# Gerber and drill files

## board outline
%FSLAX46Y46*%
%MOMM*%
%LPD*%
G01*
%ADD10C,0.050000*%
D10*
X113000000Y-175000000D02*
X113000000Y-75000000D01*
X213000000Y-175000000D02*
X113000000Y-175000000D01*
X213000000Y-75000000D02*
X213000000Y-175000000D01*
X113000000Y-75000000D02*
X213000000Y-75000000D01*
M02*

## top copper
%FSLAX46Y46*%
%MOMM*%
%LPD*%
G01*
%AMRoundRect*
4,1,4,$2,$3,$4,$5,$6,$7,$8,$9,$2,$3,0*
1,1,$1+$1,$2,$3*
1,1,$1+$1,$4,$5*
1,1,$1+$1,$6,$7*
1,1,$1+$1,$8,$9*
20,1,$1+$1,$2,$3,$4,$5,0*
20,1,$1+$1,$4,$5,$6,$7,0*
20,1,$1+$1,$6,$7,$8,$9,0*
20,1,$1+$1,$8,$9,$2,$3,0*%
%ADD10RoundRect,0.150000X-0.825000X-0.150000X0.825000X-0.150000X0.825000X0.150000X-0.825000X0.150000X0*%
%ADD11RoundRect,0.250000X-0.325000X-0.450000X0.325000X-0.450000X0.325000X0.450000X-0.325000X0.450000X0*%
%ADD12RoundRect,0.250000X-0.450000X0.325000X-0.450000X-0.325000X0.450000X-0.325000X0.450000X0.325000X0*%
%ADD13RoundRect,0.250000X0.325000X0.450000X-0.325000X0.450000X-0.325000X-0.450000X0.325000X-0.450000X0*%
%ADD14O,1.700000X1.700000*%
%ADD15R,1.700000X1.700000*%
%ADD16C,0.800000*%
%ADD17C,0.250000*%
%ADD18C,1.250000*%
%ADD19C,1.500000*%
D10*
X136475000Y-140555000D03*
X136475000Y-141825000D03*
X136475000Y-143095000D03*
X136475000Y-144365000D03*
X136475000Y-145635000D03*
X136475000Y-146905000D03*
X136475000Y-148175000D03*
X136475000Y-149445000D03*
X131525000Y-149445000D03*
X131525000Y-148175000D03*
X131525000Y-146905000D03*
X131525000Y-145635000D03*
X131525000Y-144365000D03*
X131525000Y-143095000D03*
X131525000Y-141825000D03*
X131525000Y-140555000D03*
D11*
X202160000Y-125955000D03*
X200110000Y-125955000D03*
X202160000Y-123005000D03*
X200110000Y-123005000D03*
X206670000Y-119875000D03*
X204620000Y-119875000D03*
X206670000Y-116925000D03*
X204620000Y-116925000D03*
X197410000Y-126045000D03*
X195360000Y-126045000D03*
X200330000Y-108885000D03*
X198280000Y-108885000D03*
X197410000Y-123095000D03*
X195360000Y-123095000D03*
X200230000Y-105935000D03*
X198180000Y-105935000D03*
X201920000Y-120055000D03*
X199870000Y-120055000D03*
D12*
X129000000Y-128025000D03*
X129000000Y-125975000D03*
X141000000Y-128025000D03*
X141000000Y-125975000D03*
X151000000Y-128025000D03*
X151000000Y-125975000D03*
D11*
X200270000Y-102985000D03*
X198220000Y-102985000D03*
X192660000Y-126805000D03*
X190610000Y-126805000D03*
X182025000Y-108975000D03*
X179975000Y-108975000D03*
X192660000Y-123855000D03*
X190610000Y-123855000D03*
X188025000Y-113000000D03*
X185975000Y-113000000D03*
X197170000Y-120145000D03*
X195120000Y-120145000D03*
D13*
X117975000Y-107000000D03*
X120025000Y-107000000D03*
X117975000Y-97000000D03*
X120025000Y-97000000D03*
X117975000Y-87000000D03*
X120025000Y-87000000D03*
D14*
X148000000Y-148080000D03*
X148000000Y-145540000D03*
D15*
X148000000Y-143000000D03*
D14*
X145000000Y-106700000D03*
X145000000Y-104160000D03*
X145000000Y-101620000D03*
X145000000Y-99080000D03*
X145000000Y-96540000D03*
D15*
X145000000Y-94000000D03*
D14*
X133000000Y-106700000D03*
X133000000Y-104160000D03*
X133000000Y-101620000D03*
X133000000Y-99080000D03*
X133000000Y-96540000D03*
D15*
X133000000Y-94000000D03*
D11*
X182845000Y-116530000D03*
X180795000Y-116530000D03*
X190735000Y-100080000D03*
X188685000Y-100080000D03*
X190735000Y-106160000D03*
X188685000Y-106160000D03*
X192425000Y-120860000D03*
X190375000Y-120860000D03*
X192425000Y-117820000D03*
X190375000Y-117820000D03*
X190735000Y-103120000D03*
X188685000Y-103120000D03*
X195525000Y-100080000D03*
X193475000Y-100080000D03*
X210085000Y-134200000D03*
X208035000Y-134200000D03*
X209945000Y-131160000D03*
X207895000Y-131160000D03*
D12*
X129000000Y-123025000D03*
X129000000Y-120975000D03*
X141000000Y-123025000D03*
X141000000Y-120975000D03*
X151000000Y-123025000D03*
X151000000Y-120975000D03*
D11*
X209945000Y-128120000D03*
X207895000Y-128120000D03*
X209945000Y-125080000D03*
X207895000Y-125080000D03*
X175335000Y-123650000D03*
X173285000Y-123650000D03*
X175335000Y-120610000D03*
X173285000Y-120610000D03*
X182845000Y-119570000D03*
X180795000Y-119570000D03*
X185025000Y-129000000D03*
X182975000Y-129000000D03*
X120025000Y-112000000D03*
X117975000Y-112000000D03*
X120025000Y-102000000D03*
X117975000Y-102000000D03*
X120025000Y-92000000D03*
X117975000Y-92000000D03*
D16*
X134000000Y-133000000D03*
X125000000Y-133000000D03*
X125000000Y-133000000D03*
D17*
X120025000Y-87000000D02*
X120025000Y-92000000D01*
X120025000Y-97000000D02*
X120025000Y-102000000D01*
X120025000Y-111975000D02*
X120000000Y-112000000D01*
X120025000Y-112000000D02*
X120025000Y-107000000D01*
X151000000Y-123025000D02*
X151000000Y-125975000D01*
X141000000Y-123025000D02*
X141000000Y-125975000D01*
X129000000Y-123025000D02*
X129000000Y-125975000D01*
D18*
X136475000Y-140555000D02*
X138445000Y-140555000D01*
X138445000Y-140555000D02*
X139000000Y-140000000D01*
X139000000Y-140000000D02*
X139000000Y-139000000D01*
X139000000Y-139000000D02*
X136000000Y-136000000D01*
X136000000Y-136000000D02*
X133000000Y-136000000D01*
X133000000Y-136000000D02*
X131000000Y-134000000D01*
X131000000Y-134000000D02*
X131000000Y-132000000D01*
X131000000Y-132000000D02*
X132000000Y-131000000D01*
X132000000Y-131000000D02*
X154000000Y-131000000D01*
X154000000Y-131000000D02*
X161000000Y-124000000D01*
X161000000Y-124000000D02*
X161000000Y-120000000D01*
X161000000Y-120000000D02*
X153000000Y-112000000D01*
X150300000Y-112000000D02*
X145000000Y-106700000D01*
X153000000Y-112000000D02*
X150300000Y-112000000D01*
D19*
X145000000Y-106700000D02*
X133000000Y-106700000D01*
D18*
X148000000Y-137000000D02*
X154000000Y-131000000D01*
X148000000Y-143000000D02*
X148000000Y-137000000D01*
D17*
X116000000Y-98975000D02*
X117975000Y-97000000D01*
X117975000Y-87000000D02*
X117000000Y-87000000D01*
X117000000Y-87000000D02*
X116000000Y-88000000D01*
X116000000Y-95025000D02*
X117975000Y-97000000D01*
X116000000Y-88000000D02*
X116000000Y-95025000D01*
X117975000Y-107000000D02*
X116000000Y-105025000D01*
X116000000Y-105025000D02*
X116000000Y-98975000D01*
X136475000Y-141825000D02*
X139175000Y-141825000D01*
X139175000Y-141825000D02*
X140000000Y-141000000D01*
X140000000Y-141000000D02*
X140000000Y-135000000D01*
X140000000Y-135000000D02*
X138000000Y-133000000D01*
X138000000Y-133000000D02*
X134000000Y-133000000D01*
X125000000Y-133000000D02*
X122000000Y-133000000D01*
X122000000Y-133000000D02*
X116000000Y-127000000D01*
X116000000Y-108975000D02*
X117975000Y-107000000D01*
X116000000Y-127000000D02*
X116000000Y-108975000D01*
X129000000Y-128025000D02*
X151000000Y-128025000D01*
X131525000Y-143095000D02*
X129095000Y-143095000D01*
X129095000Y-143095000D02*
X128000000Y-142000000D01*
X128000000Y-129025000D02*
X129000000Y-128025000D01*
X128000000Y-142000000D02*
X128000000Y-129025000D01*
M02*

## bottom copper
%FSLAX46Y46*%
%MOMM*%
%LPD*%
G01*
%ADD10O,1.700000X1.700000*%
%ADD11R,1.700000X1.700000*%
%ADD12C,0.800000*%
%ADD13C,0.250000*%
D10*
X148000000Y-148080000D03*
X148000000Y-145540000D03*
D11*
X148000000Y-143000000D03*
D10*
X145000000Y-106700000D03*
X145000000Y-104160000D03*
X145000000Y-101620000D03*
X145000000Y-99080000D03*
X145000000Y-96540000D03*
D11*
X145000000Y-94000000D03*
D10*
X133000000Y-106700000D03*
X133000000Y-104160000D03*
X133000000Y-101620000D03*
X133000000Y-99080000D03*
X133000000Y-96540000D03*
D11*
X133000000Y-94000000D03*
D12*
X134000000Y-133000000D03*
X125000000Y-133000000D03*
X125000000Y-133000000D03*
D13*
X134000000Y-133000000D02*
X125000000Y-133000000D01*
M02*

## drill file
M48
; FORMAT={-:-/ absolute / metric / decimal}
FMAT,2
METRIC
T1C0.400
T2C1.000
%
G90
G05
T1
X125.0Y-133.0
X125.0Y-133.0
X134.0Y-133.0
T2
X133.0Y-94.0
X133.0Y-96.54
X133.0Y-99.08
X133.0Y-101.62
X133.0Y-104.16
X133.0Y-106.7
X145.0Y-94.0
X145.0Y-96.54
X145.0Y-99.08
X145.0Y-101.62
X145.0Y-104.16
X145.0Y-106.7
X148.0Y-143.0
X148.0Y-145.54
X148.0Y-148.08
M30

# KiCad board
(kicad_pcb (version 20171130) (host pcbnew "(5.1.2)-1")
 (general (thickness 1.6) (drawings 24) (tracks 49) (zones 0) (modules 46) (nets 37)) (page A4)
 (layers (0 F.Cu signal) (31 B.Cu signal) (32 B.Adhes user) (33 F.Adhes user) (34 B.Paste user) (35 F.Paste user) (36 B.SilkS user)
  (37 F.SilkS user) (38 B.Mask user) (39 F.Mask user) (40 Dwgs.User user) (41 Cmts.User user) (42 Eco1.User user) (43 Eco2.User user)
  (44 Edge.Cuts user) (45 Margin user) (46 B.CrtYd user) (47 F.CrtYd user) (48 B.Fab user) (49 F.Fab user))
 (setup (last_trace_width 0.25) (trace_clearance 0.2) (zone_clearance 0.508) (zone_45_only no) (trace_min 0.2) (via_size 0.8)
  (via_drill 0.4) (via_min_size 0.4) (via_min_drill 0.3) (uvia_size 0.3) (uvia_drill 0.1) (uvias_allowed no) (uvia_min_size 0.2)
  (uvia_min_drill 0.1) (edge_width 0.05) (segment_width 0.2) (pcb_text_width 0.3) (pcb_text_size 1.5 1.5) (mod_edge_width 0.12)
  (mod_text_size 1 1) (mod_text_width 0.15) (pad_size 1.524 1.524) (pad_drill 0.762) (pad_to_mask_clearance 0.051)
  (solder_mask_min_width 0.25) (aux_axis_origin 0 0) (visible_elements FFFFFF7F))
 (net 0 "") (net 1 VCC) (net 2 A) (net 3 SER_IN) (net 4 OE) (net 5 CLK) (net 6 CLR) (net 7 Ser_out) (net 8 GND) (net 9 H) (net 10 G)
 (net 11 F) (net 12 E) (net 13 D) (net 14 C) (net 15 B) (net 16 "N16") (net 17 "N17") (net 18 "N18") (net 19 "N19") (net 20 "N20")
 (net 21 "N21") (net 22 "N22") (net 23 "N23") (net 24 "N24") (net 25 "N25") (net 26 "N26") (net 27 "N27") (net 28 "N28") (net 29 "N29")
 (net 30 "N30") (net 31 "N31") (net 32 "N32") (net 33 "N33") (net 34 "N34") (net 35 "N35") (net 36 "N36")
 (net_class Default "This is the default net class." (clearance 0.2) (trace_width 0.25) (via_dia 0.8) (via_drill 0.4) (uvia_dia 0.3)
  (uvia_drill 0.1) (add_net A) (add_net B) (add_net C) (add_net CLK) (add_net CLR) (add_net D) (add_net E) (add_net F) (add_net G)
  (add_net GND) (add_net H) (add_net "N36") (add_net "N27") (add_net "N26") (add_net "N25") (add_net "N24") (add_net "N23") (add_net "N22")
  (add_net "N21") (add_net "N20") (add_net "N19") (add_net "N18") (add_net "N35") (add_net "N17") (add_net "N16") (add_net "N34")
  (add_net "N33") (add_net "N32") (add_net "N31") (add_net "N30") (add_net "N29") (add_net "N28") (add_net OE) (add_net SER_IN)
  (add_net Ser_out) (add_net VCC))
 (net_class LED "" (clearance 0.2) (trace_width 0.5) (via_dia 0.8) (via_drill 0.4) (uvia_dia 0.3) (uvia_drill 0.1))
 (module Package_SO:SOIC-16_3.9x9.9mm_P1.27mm (layer F.Cu) (at 134 145)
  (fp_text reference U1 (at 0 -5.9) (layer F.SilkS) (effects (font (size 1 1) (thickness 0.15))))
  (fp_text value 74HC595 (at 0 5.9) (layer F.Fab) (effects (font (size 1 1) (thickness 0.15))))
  (pad 16 smd roundrect (at 2.475 -4.445) (size 1.95 0.6) (layers F.Cu F.Paste F.Mask) (roundrect_rratio 0.25) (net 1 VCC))
  (pad 15 smd roundrect (at 2.475 -3.175) (size 1.95 0.6) (layers F.Cu F.Paste F.Mask) (roundrect_rratio 0.25) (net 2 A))
  (pad 14 smd roundrect (at 2.475 -1.905) (size 1.95 0.6) (layers F.Cu F.Paste F.Mask) (roundrect_rratio 0.25) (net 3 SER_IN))
  (pad 13 smd roundrect (at 2.475 -0.635) (size 1.95 0.6) (layers F.Cu F.Paste F.Mask) (roundrect_rratio 0.25) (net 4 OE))
  (pad 12 smd roundrect (at 2.475 0.635) (size 1.95 0.6) (layers F.Cu F.Paste F.Mask) (roundrect_rratio 0.25) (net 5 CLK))
  (pad 11 smd roundrect (at 2.475 1.905) (size 1.95 0.6) (layers F.Cu F.Paste F.Mask) (roundrect_rratio 0.25) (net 5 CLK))
  (pad 10 smd roundrect (at 2.475 3.175) (size 1.95 0.6) (layers F.Cu F.Paste F.Mask) (roundrect_rratio 0.25) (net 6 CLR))
  (pad 9 smd roundrect (at 2.475 4.445) (size 1.95 0.6) (layers F.Cu F.Paste F.Mask) (roundrect_rratio 0.25) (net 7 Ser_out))
  (pad 8 smd roundrect (at -2.475 4.445) (size 1.95 0.6) (layers F.Cu F.Paste F.Mask) (roundrect_rratio 0.25) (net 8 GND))
  (pad 7 smd roundrect (at -2.475 3.175) (size 1.95 0.6) (layers F.Cu F.Paste F.Mask) (roundrect_rratio 0.25) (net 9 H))
  (pad 6 smd roundrect (at -2.475 1.905) (size 1.95 0.6) (layers F.Cu F.Paste F.Mask) (roundrect_rratio 0.25) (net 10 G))
  (pad 5 smd roundrect (at -2.475 0.635) (size 1.95 0.6) (layers F.Cu F.Paste F.Mask) (roundrect_rratio 0.25) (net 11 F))
  (pad 4 smd roundrect (at -2.475 -0.635) (size 1.95 0.6) (layers F.Cu F.Paste F.Mask) (roundrect_rratio 0.25) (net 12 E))
  (pad 3 smd roundrect (at -2.475 -1.905) (size 1.95 0.6) (layers F.Cu F.Paste F.Mask) (roundrect_rratio 0.25) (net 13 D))
  (pad 2 smd roundrect (at -2.475 -3.175) (size 1.95 0.6) (layers F.Cu F.Paste F.Mask) (roundrect_rratio 0.25) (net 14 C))
  (pad 1 smd roundrect (at -2.475 -4.445) (size 1.95 0.6) (layers F.Cu F.Paste F.Mask) (roundrect_rratio 0.25) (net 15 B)))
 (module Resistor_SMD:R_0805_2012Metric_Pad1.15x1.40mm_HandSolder (layer F.Cu) (at 201.135 125.955)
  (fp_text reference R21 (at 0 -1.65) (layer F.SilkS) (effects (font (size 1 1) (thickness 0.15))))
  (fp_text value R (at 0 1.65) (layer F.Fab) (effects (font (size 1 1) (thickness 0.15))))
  (pad 2 smd roundrect (at 1.025 0) (size 1.15 1.4) (layers F.Cu F.Paste F.Mask) (roundrect_rratio 0.217391) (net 10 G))
  (pad 1 smd roundrect (at -1.025 0) (size 1.15 1.4) (layers F.Cu F.Paste F.Mask) (roundrect_rratio 0.217391) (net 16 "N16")))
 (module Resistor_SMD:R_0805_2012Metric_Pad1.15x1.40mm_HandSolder (layer F.Cu) (at 201.135 123.005)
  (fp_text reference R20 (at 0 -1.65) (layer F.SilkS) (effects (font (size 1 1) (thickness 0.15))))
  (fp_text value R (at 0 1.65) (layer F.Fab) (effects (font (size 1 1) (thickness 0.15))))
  (pad 2 smd roundrect (at 1.025 0) (size 1.15 1.4) (layers F.Cu F.Paste F.Mask) (roundrect_rratio 0.217391) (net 10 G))
  (pad 1 smd roundrect (at -1.025 0) (size 1.15 1.4) (layers F.Cu F.Paste F.Mask) (roundrect_rratio 0.217391) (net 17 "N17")))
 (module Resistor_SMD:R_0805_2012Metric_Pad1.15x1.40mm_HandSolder (layer F.Cu) (at 205.645 119.875)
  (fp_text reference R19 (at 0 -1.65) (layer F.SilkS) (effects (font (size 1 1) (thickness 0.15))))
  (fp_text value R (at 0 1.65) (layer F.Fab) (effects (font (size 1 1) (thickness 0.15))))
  (pad 2 smd roundrect (at 1.025 0) (size 1.15 1.4) (layers F.Cu F.Paste F.Mask) (roundrect_rratio 0.217391) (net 10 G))
  (pad 1 smd roundrect (at -1.025 0) (size 1.15 1.4) (layers F.Cu F.Paste F.Mask) (roundrect_rratio 0.217391) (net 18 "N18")))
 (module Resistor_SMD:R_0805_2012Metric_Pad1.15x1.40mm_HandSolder (layer F.Cu) (at 205.645 116.925)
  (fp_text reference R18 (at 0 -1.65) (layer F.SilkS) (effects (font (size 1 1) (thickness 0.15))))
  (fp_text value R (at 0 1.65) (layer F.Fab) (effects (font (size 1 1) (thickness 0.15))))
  (pad 2 smd roundrect (at 1.025 0) (size 1.15 1.4) (layers F.Cu F.Paste F.Mask) (roundrect_rratio 0.217391) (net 11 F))
  (pad 1 smd roundrect (at -1.025 0) (size 1.15 1.4) (layers F.Cu F.Paste F.Mask) (roundrect_rratio 0.217391) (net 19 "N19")))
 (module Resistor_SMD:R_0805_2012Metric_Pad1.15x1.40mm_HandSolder (layer F.Cu) (at 196.385 126.045)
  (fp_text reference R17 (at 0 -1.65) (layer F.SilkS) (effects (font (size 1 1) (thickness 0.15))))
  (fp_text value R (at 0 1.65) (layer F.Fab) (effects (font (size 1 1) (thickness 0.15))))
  (pad 2 smd roundrect (at 1.025 0) (size 1.15 1.4) (layers F.Cu F.Paste F.Mask) (roundrect_rratio 0.217391) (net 11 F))
  (pad 1 smd roundrect (at -1.025 0) (size 1.15 1.4) (layers F.Cu F.Paste F.Mask) (roundrect_rratio 0.217391) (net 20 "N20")))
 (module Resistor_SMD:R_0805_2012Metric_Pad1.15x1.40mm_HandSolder (layer F.Cu) (at 199.305 108.885)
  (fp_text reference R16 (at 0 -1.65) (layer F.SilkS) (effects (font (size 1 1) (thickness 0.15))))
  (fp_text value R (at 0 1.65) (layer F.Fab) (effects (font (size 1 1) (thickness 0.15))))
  (pad 2 smd roundrect (at 1.025 0) (size 1.15 1.4) (layers F.Cu F.Paste F.Mask) (roundrect_rratio 0.217391) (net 11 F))
  (pad 1 smd roundrect (at -1.025 0) (size 1.15 1.4) (layers F.Cu F.Paste F.Mask) (roundrect_rratio 0.217391) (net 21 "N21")))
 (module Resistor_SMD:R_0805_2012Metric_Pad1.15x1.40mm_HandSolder (layer F.Cu) (at 196.385 123.095)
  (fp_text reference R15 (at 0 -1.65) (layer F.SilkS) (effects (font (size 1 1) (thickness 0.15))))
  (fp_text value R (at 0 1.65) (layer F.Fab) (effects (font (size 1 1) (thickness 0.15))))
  (pad 2 smd roundrect (at 1.025 0) (size 1.15 1.4) (layers F.Cu F.Paste F.Mask) (roundrect_rratio 0.217391) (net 12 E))
  (pad 1 smd roundrect (at -1.025 0) (size 1.15 1.4) (layers F.Cu F.Paste F.Mask) (roundrect_rratio 0.217391) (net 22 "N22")))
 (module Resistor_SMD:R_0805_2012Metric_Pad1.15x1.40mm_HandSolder (layer F.Cu) (at 199.205 105.935)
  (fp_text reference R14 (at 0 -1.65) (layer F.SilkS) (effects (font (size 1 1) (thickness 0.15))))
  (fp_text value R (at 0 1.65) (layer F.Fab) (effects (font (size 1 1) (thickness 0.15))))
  (pad 2 smd roundrect (at 1.025 0) (size 1.15 1.4) (layers F.Cu F.Paste F.Mask) (roundrect_rratio 0.217391) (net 12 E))
  (pad 1 smd roundrect (at -1.025 0) (size 1.15 1.4) (layers F.Cu F.Paste F.Mask) (roundrect_rratio 0.217391) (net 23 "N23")))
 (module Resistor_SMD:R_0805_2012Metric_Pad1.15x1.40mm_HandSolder (layer F.Cu) (at 200.895 120.055)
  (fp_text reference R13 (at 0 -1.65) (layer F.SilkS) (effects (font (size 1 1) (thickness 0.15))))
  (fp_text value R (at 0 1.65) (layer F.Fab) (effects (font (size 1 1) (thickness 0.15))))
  (pad 2 smd roundrect (at 1.025 0) (size 1.15 1.4) (layers F.Cu F.Paste F.Mask) (roundrect_rratio 0.217391) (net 12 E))
  (pad 1 smd roundrect (at -1.025 0) (size 1.15 1.4) (layers F.Cu F.Paste F.Mask) (roundrect_rratio 0.217391) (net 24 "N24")))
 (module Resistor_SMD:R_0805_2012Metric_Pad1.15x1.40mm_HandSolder (layer F.Cu) (at 129 127 270)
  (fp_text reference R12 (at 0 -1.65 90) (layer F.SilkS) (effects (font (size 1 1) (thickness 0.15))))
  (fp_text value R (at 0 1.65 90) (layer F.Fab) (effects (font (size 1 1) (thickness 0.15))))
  (pad 2 smd roundrect (at 1.025 0 270) (size 1.15 1.4) (layers F.Cu F.Paste F.Mask) (roundrect_rratio 0.217391) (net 13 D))
  (pad 1 smd roundrect (at -1.025 0 270) (size 1.15 1.4) (layers F.Cu F.Paste F.Mask) (roundrect_rratio 0.217391) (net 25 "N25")))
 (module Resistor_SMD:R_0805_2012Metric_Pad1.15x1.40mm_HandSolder (layer F.Cu) (at 141 127 270)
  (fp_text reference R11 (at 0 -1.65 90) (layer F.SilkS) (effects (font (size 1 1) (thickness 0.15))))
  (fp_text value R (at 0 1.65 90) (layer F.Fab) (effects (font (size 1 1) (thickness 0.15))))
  (pad 2 smd roundrect (at 1.025 0 270) (size 1.15 1.4) (layers F.Cu F.Paste F.Mask) (roundrect_rratio 0.217391) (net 13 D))
  (pad 1 smd roundrect (at -1.025 0 270) (size 1.15 1.4) (layers F.Cu F.Paste F.Mask) (roundrect_rratio 0.217391) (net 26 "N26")))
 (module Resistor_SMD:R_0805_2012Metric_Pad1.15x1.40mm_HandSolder (layer F.Cu) (at 151 127 270)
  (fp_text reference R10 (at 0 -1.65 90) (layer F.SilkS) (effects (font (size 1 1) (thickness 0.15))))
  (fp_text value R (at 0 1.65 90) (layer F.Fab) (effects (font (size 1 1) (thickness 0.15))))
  (pad 2 smd roundrect (at 1.025 0 270) (size 1.15 1.4) (layers F.Cu F.Paste F.Mask) (roundrect_rratio 0.217391) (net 13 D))
  (pad 1 smd roundrect (at -1.025 0 270) (size 1.15 1.4) (layers F.Cu F.Paste F.Mask) (roundrect_rratio 0.217391) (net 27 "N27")))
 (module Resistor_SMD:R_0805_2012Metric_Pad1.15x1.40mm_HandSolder (layer F.Cu) (at 199.245 102.985)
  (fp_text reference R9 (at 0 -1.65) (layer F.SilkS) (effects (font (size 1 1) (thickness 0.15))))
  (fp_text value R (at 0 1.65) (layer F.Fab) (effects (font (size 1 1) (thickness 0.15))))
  (pad 2 smd roundrect (at 1.025 0) (size 1.15 1.4) (layers F.Cu F.Paste F.Mask) (roundrect_rratio 0.217391) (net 14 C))
  (pad 1 smd roundrect (at -1.025 0) (size 1.15 1.4) (layers F.Cu F.Paste F.Mask) (roundrect_rratio 0.217391) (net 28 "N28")))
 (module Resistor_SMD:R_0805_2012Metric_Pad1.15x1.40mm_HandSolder (layer F.Cu) (at 191.635 126.805)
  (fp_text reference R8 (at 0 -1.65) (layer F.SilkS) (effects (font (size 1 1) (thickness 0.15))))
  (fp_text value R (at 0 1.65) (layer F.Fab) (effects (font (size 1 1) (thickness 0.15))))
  (pad 2 smd roundrect (at 1.025 0) (size 1.15 1.4) (layers F.Cu F.Paste F.Mask) (roundrect_rratio 0.217391) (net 14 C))
  (pad 1 smd roundrect (at -1.025 0) (size 1.15 1.4) (layers F.Cu F.Paste F.Mask) (roundrect_rratio 0.217391) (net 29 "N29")))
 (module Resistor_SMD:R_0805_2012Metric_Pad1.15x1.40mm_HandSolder (layer F.Cu) (at 181 108.975)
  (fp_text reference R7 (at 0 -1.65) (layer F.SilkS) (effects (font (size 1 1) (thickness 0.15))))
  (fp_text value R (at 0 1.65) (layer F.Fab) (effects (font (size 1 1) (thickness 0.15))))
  (pad 2 smd roundrect (at 1.025 0) (size 1.15 1.4) (layers F.Cu F.Paste F.Mask) (roundrect_rratio 0.217391) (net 14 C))
  (pad 1 smd roundrect (at -1.025 0) (size 1.15 1.4) (layers F.Cu F.Paste F.Mask) (roundrect_rratio 0.217391) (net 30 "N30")))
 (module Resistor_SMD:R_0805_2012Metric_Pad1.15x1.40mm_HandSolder (layer F.Cu) (at 191.635 123.855)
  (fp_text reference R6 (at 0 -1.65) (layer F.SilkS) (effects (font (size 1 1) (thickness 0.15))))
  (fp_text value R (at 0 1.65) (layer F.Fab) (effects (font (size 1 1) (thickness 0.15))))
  (pad 2 smd roundrect (at 1.025 0) (size 1.15 1.4) (layers F.Cu F.Paste F.Mask) (roundrect_rratio 0.217391) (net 15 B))
  (pad 1 smd roundrect (at -1.025 0) (size 1.15 1.4) (layers F.Cu F.Paste F.Mask) (roundrect_rratio 0.217391) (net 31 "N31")))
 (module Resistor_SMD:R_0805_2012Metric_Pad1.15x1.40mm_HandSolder (layer F.Cu) (at 187 113)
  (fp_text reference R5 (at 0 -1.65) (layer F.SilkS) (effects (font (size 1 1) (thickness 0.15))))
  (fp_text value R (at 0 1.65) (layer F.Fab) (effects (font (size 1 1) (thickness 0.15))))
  (pad 2 smd roundrect (at 1.025 0) (size 1.15 1.4) (layers F.Cu F.Paste F.Mask) (roundrect_rratio 0.217391) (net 15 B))
  (pad 1 smd roundrect (at -1.025 0) (size 1.15 1.4) (layers F.Cu F.Paste F.Mask) (roundrect_rratio 0.217391) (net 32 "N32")))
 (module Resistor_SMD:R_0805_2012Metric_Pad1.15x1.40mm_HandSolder (layer F.Cu) (at 196.145 120.145)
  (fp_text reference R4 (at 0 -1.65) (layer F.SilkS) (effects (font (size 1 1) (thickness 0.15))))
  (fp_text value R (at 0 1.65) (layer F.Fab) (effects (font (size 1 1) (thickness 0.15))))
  (pad 2 smd roundrect (at 1.025 0) (size 1.15 1.4) (layers F.Cu F.Paste F.Mask) (roundrect_rratio 0.217391) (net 15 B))
  (pad 1 smd roundrect (at -1.025 0) (size 1.15 1.4) (layers F.Cu F.Paste F.Mask) (roundrect_rratio 0.217391) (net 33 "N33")))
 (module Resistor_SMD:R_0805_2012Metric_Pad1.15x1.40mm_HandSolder (layer F.Cu) (at 119 107 180)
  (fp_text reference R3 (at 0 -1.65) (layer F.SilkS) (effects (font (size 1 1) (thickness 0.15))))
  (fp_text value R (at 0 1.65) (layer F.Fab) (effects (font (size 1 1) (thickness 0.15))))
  (pad 2 smd roundrect (at 1.025 0 180) (size 1.15 1.4) (layers F.Cu F.Paste F.Mask) (roundrect_rratio 0.217391) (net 2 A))
  (pad 1 smd roundrect (at -1.025 0 180) (size 1.15 1.4) (layers F.Cu F.Paste F.Mask) (roundrect_rratio 0.217391) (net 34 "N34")))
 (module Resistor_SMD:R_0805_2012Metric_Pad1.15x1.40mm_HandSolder (layer F.Cu) (at 119 97 180)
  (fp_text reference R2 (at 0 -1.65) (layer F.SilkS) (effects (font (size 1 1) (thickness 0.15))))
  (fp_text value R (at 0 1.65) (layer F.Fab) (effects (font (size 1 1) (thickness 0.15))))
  (pad 2 smd roundrect (at 1.025 0 180) (size 1.15 1.4) (layers F.Cu F.Paste F.Mask) (roundrect_rratio 0.217391) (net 2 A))
  (pad 1 smd roundrect (at -1.025 0 180) (size 1.15 1.4) (layers F.Cu F.Paste F.Mask) (roundrect_rratio 0.217391) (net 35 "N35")))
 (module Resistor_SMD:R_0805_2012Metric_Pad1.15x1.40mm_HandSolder (layer F.Cu) (at 119 87 180)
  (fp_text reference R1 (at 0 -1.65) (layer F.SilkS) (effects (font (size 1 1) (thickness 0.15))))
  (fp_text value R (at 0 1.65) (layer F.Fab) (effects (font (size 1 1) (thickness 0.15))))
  (pad 2 smd roundrect (at 1.025 0 180) (size 1.15 1.4) (layers F.Cu F.Paste F.Mask) (roundrect_rratio 0.217391) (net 2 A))
  (pad 1 smd roundrect (at -1.025 0 180) (size 1.15 1.4) (layers F.Cu F.Paste F.Mask) (roundrect_rratio 0.217391) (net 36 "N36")))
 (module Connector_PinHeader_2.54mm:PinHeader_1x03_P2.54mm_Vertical (layer F.Cu) (at 148 143)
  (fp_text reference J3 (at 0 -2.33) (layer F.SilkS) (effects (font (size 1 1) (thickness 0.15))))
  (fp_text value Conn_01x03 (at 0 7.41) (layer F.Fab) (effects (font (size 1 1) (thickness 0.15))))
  (pad 3 thru_hole oval (at 0 5.08) (size 1.7 1.7) (drill 1) (layers *.Cu *.Mask) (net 9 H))
  (pad 2 thru_hole oval (at 0 2.54) (size 1.7 1.7) (drill 1) (layers *.Cu *.Mask) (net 8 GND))
  (pad 1 thru_hole rect (at 0 0) (size 1.7 1.7) (drill 1) (layers *.Cu *.Mask) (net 1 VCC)))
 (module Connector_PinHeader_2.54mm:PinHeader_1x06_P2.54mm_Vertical (layer F.Cu) (at 145 94)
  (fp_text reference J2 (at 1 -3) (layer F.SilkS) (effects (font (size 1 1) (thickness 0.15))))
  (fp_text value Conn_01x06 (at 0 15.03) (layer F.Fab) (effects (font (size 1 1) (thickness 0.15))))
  (pad 6 thru_hole oval (at 0 12.7) (size 1.7 1.7) (drill 1) (layers *.Cu *.Mask) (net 1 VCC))
  (pad 5 thru_hole oval (at 0 10.16) (size 1.7 1.7) (drill 1) (layers *.Cu *.Mask) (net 8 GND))
  (pad 4 thru_hole oval (at 0 7.62) (size 1.7 1.7) (drill 1) (layers *.Cu *.Mask) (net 7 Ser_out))
  (pad 3 thru_hole oval (at 0 5.08) (size 1.7 1.7) (drill 1) (layers *.Cu *.Mask) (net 5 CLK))
  (pad 2 thru_hole oval (at 0 2.54) (size 1.7 1.7) (drill 1) (layers *.Cu *.Mask) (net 4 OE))
  (pad 1 thru_hole rect (at 0 0) (size 1.7 1.7) (drill 1) (layers *.Cu *.Mask) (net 6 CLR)))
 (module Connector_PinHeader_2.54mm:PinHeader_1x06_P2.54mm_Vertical (layer F.Cu) (at 133 94)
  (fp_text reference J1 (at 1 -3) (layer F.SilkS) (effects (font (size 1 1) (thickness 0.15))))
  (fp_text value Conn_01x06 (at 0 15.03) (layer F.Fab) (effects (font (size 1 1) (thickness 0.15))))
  (pad 6 thru_hole oval (at 0 12.7) (size 1.7 1.7) (drill 1) (layers *.Cu *.Mask) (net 1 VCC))
  (pad 5 thru_hole oval (at 0 10.16) (size 1.7 1.7) (drill 1) (layers *.Cu *.Mask) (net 8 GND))
  (pad 4 thru_hole oval (at 0 7.62) (size 1.7 1.7) (drill 1) (layers *.Cu *.Mask) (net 3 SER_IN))
  (pad 3 thru_hole oval (at 0 5.08) (size 1.7 1.7) (drill 1) (layers *.Cu *.Mask) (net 5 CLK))
  (pad 2 thru_hole oval (at 0 2.54) (size 1.7 1.7) (drill 1) (layers *.Cu *.Mask) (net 4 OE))
  (pad 1 thru_hole rect (at 0 0) (size 1.7 1.7) (drill 1) (layers *.Cu *.Mask) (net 6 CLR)))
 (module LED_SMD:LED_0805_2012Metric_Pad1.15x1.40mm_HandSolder (layer F.Cu) (at 181.82 116.53)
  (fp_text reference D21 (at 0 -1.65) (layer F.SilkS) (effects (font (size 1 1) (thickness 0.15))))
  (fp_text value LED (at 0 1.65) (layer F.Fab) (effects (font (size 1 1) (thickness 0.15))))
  (pad 2 smd roundrect (at 1.025 0) (size 1.15 1.4) (layers F.Cu F.Paste F.Mask) (roundrect_rratio 0.217391) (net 16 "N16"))
  (pad 1 smd roundrect (at -1.025 0) (size 1.15 1.4) (layers F.Cu F.Paste F.Mask) (roundrect_rratio 0.217391) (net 8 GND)))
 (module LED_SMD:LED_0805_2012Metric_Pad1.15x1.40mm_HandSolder (layer F.Cu) (at 189.71 100.08)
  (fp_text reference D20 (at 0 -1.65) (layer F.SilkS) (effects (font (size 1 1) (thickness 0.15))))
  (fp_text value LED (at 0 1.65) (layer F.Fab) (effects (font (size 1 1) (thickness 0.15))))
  (pad 2 smd roundrect (at 1.025 0) (size 1.15 1.4) (layers F.Cu F.Paste F.Mask) (roundrect_rratio 0.217391) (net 17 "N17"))
  (pad 1 smd roundrect (at -1.025 0) (size 1.15 1.4) (layers F.Cu F.Paste F.Mask) (roundrect_rratio 0.217391) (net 8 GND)))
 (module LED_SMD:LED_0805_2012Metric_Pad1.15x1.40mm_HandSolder (layer F.Cu) (at 189.71 106.16)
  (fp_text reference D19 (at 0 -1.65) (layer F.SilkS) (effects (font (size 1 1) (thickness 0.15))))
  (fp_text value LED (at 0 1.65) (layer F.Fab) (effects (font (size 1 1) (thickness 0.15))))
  (pad 2 smd roundrect (at 1.025 0) (size 1.15 1.4) (layers F.Cu F.Paste F.Mask) (roundrect_rratio 0.217391) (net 18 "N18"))
  (pad 1 smd roundrect (at -1.025 0) (size 1.15 1.4) (layers F.Cu F.Paste F.Mask) (roundrect_rratio 0.217391) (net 8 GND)))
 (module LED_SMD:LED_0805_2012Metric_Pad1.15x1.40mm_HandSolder (layer F.Cu) (at 191.4 120.86)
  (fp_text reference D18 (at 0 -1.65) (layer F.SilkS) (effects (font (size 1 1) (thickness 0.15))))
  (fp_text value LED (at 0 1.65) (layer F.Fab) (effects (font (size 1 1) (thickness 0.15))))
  (pad 2 smd roundrect (at 1.025 0) (size 1.15 1.4) (layers F.Cu F.Paste F.Mask) (roundrect_rratio 0.217391) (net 19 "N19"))
  (pad 1 smd roundrect (at -1.025 0) (size 1.15 1.4) (layers F.Cu F.Paste F.Mask) (roundrect_rratio 0.217391) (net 8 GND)))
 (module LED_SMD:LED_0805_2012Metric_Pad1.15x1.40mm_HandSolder (layer F.Cu) (at 191.4 117.82)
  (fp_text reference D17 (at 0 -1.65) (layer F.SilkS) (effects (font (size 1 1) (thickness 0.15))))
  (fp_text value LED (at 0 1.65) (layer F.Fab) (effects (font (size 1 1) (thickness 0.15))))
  (pad 2 smd roundrect (at 1.025 0) (size 1.15 1.4) (layers F.Cu F.Paste F.Mask) (roundrect_rratio 0.217391) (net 20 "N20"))
  (pad 1 smd roundrect (at -1.025 0) (size 1.15 1.4) (layers F.Cu F.Paste F.Mask) (roundrect_rratio 0.217391) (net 8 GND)))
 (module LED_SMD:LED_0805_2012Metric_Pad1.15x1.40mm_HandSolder (layer F.Cu) (at 189.71 103.12)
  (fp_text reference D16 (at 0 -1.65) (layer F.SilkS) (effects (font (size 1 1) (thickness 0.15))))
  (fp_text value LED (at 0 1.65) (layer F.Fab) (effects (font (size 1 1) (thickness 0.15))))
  (pad 2 smd roundrect (at 1.025 0) (size 1.15 1.4) (layers F.Cu F.Paste F.Mask) (roundrect_rratio 0.217391) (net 21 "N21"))
  (pad 1 smd roundrect (at -1.025 0) (size 1.15 1.4) (layers F.Cu F.Paste F.Mask) (roundrect_rratio 0.217391) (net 8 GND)))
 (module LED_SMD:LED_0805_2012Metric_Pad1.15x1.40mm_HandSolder (layer F.Cu) (at 194.5 100.08)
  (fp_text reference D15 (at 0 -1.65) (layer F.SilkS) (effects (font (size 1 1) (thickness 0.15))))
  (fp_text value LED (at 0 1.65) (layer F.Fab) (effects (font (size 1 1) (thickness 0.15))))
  (pad 2 smd roundrect (at 1.025 0) (size 1.15 1.4) (layers F.Cu F.Paste F.Mask) (roundrect_rratio 0.217391) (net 22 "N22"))
  (pad 1 smd roundrect (at -1.025 0) (size 1.15 1.4) (layers F.Cu F.Paste F.Mask) (roundrect_rratio 0.217391) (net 8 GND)))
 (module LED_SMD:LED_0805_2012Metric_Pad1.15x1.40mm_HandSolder (layer F.Cu) (at 209.06 134.2)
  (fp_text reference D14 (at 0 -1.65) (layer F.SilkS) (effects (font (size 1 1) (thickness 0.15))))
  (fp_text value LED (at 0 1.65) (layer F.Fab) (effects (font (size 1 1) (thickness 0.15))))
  (pad 2 smd roundrect (at 1.025 0) (size 1.15 1.4) (layers F.Cu F.Paste F.Mask) (roundrect_rratio 0.217391) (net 23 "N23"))
  (pad 1 smd roundrect (at -1.025 0) (size 1.15 1.4) (layers F.Cu F.Paste F.Mask) (roundrect_rratio 0.217391) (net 8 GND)))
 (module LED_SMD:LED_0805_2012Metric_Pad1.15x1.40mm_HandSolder (layer F.Cu) (at 208.92 131.16)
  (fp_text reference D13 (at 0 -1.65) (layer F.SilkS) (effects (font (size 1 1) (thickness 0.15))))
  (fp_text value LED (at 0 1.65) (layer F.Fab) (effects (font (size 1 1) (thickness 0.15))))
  (pad 2 smd roundrect (at 1.025 0) (size 1.15 1.4) (layers F.Cu F.Paste F.Mask) (roundrect_rratio 0.217391) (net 24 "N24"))
  (pad 1 smd roundrect (at -1.025 0) (size 1.15 1.4) (layers F.Cu F.Paste F.Mask) (roundrect_rratio 0.217391) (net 8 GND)))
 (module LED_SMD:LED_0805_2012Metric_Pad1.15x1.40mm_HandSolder (layer F.Cu) (at 129 122 270)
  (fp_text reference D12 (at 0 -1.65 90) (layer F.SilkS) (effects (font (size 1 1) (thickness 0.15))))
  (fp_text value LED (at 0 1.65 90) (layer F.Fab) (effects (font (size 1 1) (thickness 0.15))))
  (pad 2 smd roundrect (at 1.025 0 270) (size 1.15 1.4) (layers F.Cu F.Paste F.Mask) (roundrect_rratio 0.217391) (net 25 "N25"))
  (pad 1 smd roundrect (at -1.025 0 270) (size 1.15 1.4) (layers F.Cu F.Paste F.Mask) (roundrect_rratio 0.217391) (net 8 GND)))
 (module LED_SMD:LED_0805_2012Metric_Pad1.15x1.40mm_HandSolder (layer F.Cu) (at 141 122 270)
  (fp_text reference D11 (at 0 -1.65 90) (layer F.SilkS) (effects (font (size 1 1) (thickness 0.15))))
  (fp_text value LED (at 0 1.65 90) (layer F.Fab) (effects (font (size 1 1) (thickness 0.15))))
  (pad 2 smd roundrect (at 1.025 0 270) (size 1.15 1.4) (layers F.Cu F.Paste F.Mask) (roundrect_rratio 0.217391) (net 26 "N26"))
  (pad 1 smd roundrect (at -1.025 0 270) (size 1.15 1.4) (layers F.Cu F.Paste F.Mask) (roundrect_rratio 0.217391) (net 8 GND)))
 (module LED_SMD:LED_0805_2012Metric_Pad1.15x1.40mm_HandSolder (layer F.Cu) (at 151 122 270)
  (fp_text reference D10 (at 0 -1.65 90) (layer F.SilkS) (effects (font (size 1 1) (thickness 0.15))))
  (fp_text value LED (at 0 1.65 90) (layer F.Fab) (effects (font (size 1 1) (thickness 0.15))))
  (pad 2 smd roundrect (at 1.025 0 270) (size 1.15 1.4) (layers F.Cu F.Paste F.Mask) (roundrect_rratio 0.217391) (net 27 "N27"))
  (pad 1 smd roundrect (at -1.025 0 270) (size 1.15 1.4) (layers F.Cu F.Paste F.Mask) (roundrect_rratio 0.217391) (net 8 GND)))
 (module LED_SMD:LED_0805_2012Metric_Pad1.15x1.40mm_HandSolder (layer F.Cu) (at 208.92 128.12)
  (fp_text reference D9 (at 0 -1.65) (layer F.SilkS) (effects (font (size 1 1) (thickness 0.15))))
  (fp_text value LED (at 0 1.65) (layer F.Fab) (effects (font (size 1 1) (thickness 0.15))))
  (pad 2 smd roundrect (at 1.025 0) (size 1.15 1.4) (layers F.Cu F.Paste F.Mask) (roundrect_rratio 0.217391) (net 28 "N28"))
  (pad 1 smd roundrect (at -1.025 0) (size 1.15 1.4) (layers F.Cu F.Paste F.Mask) (roundrect_rratio 0.217391) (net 8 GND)))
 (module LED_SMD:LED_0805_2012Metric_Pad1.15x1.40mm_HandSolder (layer F.Cu) (at 208.92 125.08)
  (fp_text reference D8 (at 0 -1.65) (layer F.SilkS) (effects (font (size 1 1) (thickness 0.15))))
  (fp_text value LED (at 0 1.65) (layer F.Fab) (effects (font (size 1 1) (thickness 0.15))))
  (pad 2 smd roundrect (at 1.025 0) (size 1.15 1.4) (layers F.Cu F.Paste F.Mask) (roundrect_rratio 0.217391) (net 29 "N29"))
  (pad 1 smd roundrect (at -1.025 0) (size 1.15 1.4) (layers F.Cu F.Paste F.Mask) (roundrect_rratio 0.217391) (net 8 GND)))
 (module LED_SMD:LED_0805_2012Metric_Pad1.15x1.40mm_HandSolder (layer F.Cu) (at 174.31 123.65)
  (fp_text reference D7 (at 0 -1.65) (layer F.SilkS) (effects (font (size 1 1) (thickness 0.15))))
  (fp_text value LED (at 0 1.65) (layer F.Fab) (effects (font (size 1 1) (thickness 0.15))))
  (pad 2 smd roundrect (at 1.025 0) (size 1.15 1.4) (layers F.Cu F.Paste F.Mask) (roundrect_rratio 0.217391) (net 30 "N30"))
  (pad 1 smd roundrect (at -1.025 0) (size 1.15 1.4) (layers F.Cu F.Paste F.Mask) (roundrect_rratio 0.217391) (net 8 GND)))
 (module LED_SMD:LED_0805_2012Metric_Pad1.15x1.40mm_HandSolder (layer F.Cu) (at 174.31 120.61)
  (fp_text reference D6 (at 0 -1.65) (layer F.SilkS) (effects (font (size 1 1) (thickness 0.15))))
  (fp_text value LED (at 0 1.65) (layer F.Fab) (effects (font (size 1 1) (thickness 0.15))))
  (pad 2 smd roundrect (at 1.025 0) (size 1.15 1.4) (layers F.Cu F.Paste F.Mask) (roundrect_rratio 0.217391) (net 31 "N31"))
  (pad 1 smd roundrect (at -1.025 0) (size 1.15 1.4) (layers F.Cu F.Paste F.Mask) (roundrect_rratio 0.217391) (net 8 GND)))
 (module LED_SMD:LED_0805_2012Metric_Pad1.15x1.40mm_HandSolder (layer F.Cu) (at 181.82 119.57)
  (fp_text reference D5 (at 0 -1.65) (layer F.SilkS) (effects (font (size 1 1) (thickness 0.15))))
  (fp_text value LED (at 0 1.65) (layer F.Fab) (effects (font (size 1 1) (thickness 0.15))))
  (pad 2 smd roundrect (at 1.025 0) (size 1.15 1.4) (layers F.Cu F.Paste F.Mask) (roundrect_rratio 0.217391) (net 32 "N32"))
  (pad 1 smd roundrect (at -1.025 0) (size 1.15 1.4) (layers F.Cu F.Paste F.Mask) (roundrect_rratio 0.217391) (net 8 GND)))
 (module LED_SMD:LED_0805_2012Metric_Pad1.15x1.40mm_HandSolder (layer F.Cu) (at 184 129)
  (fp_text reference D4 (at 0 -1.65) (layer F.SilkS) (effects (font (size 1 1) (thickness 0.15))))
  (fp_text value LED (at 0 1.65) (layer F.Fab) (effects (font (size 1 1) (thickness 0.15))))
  (pad 2 smd roundrect (at 1.025 0) (size 1.15 1.4) (layers F.Cu F.Paste F.Mask) (roundrect_rratio 0.217391) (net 33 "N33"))
  (pad 1 smd roundrect (at -1.025 0) (size 1.15 1.4) (layers F.Cu F.Paste F.Mask) (roundrect_rratio 0.217391) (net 8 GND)))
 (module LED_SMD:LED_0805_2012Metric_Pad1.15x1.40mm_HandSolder (layer F.Cu) (at 119 112)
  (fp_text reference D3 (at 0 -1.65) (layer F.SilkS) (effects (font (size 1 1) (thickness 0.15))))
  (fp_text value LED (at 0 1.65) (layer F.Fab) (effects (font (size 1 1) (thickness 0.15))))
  (pad 2 smd roundrect (at 1.025 0) (size 1.15 1.4) (layers F.Cu F.Paste F.Mask) (roundrect_rratio 0.217391) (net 34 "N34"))
  (pad 1 smd roundrect (at -1.025 0) (size 1.15 1.4) (layers F.Cu F.Paste F.Mask) (roundrect_rratio 0.217391) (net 8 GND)))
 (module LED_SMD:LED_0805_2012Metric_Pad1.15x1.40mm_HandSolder (layer F.Cu) (at 119 102)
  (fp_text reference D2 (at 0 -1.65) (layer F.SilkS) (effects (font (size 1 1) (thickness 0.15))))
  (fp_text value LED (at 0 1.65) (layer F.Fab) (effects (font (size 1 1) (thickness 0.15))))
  (pad 2 smd roundrect (at 1.025 0) (size 1.15 1.4) (layers F.Cu F.Paste F.Mask) (roundrect_rratio 0.217391) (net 35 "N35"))
  (pad 1 smd roundrect (at -1.025 0) (size 1.15 1.4) (layers F.Cu F.Paste F.Mask) (roundrect_rratio 0.217391) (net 8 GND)))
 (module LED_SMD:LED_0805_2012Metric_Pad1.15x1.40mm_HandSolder (layer F.Cu) (at 119 92)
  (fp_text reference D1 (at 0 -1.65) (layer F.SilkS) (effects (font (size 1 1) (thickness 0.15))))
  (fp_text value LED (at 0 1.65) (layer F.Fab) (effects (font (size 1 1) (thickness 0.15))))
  (pad 2 smd roundrect (at 1.025 0) (size 1.15 1.4) (layers F.Cu F.Paste F.Mask) (roundrect_rratio 0.217391) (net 36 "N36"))
  (pad 1 smd roundrect (at -1.025 0) (size 1.15 1.4) (layers F.Cu F.Paste F.Mask) (roundrect_rratio 0.217391) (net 8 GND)))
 (gr_line (start 113 175) (end 113 75) (layer Edge.Cuts) (width 0.05))
 (gr_line (start 213 175) (end 113 175) (layer Edge.Cuts) (width 0.05))
 (gr_line (start 213 75) (end 213 175) (layer Edge.Cuts) (width 0.05))
 (gr_line (start 113 75) (end 213 75) (layer Edge.Cuts) (width 0.05))
 (segment (start 120.025 87) (end 120.025 92) (width 0.25) (layer F.Cu) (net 36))
 (segment (start 120.025 97) (end 120.025 102) (width 0.25) (layer F.Cu) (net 35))
 (segment (start 120.025 111.975) (end 120 112) (width 0.25) (layer F.Cu) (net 34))
 (segment (start 120.025 112) (end 120.025 107) (width 0.25) (layer F.Cu) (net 34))
 (segment (start 151 123.025) (end 151 125.975) (width 0.25) (layer F.Cu) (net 27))
 (segment (start 141 123.025) (end 141 125.975) (width 0.25) (layer F.Cu) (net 26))
 (segment (start 129 123.025) (end 129 125.975) (width 0.25) (layer F.Cu) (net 25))
 (segment (start 136.475 140.555) (end 138.445 140.555) (width 1.25) (layer F.Cu) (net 1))
 (segment (start 138.445 140.555) (end 139 140) (width 1.25) (layer F.Cu) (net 1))
 (segment (start 139 140) (end 139 139) (width 1.25) (layer F.Cu) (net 1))
 (segment (start 139 139) (end 136 136) (width 1.25) (layer F.Cu) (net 1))
 (segment (start 136 136) (end 133 136) (width 1.25) (layer F.Cu) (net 1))
 (segment (start 133 136) (end 131 134) (width 1.25) (layer F.Cu) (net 1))
 (segment (start 131 134) (end 131 132) (width 1.25) (layer F.Cu) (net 1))
 (segment (start 131 132) (end 132 131) (width 1.25) (layer F.Cu) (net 1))
 (segment (start 132 131) (end 154 131) (width 1.25) (layer F.Cu) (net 1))
 (segment (start 154 131) (end 161 124) (width 1.25) (layer F.Cu) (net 1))
 (segment (start 161 124) (end 161 120) (width 1.25) (layer F.Cu) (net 1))
 (segment (start 161 120) (end 153 112) (width 1.25) (layer F.Cu) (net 1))
 (segment (start 150.3 112) (end 145 106.7) (width 1.25) (layer F.Cu) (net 1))
 (segment (start 153 112) (end 150.3 112) (width 1.25) (layer F.Cu) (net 1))
 (segment (start 145 106.7) (end 133 106.7) (width 1.5) (layer F.Cu) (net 1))
 (segment (start 148 137) (end 154 131) (width 1.25) (layer F.Cu) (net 1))
 (segment (start 148 143) (end 148 137) (width 1.25) (layer F.Cu) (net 1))
 (segment (start 116 98.975) (end 117.975 97) (width 0.25) (layer F.Cu) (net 2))
 (segment (start 117.975 87) (end 117 87) (width 0.25) (layer F.Cu) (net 2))
 (segment (start 117 87) (end 116 88) (width 0.25) (layer F.Cu) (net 2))
 (segment (start 116 95.025) (end 117.975 97) (width 0.25) (layer F.Cu) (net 2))
 (segment (start 116 88) (end 116 95.025) (width 0.25) (layer F.Cu) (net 2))
 (segment (start 117.975 107) (end 116 105.025) (width 0.25) (layer F.Cu) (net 2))
 (segment (start 116 105.025) (end 116 98.975) (width 0.25) (layer F.Cu) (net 2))
 (segment (start 136.475 141.825) (end 139.175 141.825) (width 0.25) (layer F.Cu) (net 2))
 (segment (start 139.175 141.825) (end 140 141) (width 0.25) (layer F.Cu) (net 2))
 (segment (start 140 141) (end 140 135) (width 0.25) (layer F.Cu) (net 2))
 (segment (start 140 135) (end 138 133) (width 0.25) (layer F.Cu) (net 2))
 (via (at 134 133) (size 0.8) (drill 0.4) (layers F.Cu B.Cu) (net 2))
 (segment (start 138 133) (end 134 133) (width 0.25) (layer F.Cu) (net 2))
 (segment (start 134 133) (end 125 133) (width 0.25) (layer B.Cu) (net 2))
 (via (at 125 133) (size 0.8) (drill 0.4) (layers F.Cu B.Cu) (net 2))
 (via (at 125 133) (size 0.8) (drill 0.4) (layers F.Cu B.Cu) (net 2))
 (segment (start 125 133) (end 122 133) (width 0.25) (layer F.Cu) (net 2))
 (segment (start 122 133) (end 116 127) (width 0.25) (layer F.Cu) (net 2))
 (segment (start 116 108.975) (end 117.975 107) (width 0.25) (layer F.Cu) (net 2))
 (segment (start 116 127) (end 116 108.975) (width 0.25) (layer F.Cu) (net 2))
 (segment (start 129 128.025) (end 151 128.025) (width 0.25) (layer F.Cu) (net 13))
 (segment (start 131.525 143.095) (end 129.095 143.095) (width 0.25) (layer F.Cu) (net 13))
 (segment (start 129.095 143.095) (end 128 142) (width 0.25) (layer F.Cu) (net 13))
 (segment (start 128 129.025) (end 129 128.025) (width 0.25) (layer F.Cu) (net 13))
 (segment (start 128 142) (end 128 129.025) (width 0.25) (layer F.Cu) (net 13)))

